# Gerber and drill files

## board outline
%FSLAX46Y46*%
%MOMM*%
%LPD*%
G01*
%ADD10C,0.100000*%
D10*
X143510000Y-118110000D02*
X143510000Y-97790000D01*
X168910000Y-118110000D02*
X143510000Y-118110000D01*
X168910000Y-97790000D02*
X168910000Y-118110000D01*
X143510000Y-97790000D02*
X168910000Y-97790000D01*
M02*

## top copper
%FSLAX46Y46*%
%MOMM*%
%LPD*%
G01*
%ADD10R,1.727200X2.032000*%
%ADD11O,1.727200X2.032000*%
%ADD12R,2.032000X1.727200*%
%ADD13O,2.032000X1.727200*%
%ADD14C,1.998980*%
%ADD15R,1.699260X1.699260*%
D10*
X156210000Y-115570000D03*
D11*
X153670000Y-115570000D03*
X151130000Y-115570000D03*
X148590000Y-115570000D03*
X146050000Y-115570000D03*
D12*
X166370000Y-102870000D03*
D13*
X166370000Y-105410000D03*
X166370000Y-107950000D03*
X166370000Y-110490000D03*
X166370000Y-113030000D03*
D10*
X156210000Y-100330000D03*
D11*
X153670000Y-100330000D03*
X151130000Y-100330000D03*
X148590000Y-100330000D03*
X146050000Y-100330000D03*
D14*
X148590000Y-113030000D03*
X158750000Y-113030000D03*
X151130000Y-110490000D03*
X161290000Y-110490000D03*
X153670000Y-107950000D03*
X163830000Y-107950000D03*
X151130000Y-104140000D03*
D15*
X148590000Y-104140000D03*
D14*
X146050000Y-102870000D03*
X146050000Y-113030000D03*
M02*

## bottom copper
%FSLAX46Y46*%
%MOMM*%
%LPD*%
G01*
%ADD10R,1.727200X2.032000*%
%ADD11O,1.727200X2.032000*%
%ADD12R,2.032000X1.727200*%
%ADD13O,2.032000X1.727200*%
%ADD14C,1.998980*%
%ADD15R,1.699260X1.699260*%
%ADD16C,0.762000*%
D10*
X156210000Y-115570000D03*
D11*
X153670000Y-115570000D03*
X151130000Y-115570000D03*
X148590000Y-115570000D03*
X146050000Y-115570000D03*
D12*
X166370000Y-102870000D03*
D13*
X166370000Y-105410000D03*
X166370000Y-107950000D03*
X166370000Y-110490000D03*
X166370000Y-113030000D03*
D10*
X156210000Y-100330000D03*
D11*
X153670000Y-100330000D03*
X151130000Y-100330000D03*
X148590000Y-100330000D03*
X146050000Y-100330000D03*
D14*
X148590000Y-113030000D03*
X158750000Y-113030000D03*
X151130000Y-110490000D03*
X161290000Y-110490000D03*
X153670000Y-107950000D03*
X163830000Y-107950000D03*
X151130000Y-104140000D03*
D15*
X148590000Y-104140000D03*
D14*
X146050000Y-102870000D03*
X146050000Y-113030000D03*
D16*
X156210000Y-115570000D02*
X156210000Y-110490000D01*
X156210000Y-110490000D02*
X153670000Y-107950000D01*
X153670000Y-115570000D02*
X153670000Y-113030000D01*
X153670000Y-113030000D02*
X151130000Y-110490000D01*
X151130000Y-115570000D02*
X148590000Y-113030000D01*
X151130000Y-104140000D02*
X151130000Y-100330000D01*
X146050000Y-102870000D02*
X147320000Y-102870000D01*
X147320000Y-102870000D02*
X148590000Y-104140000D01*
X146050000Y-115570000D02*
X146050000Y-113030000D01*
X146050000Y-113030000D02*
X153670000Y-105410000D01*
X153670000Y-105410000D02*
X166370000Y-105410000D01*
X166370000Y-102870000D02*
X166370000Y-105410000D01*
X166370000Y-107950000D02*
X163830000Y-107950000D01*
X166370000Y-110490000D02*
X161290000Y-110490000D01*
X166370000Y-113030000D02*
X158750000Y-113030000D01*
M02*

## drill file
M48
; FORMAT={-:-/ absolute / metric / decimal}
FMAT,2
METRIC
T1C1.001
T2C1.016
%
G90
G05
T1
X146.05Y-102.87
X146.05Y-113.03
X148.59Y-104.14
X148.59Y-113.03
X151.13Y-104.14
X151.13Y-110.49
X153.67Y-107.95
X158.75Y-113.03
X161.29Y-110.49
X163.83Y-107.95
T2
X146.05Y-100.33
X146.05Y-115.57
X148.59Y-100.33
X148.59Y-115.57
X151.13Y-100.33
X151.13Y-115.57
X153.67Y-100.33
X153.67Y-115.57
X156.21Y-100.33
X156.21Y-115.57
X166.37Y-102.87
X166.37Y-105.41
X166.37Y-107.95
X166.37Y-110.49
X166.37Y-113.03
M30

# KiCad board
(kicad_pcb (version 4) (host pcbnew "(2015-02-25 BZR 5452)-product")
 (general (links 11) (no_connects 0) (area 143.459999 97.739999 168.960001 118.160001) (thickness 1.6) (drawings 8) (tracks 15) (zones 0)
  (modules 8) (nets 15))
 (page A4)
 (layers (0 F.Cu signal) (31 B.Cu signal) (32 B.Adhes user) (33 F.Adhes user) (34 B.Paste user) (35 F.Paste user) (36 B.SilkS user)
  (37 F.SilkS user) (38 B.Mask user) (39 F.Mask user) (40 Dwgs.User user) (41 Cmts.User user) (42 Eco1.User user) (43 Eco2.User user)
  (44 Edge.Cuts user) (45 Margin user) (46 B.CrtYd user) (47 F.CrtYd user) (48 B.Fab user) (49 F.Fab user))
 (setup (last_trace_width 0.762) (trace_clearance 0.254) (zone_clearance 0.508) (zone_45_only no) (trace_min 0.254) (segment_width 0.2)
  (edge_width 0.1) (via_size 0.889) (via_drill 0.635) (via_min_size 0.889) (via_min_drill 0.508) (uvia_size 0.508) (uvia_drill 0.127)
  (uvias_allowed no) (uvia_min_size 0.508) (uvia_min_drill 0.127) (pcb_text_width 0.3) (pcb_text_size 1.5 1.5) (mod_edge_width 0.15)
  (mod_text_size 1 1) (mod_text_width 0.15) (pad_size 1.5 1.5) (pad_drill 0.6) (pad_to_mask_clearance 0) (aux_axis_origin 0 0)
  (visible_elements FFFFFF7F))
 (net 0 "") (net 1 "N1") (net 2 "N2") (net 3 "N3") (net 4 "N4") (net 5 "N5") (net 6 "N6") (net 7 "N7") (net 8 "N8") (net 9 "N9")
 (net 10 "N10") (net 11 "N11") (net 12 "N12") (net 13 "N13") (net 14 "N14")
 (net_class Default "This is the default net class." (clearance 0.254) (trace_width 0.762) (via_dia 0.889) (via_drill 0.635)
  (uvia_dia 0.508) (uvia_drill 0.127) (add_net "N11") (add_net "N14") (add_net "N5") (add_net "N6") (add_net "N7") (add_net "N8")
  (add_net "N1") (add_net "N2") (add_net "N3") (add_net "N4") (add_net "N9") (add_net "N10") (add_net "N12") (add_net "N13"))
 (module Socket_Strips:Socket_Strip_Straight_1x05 (layer F.Cu) (at 156.21 115.57 180)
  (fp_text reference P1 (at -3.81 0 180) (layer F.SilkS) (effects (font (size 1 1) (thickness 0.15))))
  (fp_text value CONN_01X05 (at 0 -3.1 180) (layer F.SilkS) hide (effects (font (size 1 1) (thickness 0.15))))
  (pad 1 thru_hole rect (at 0 0 180) (size 1.7272 2.032) (drill 1.016) (layers *.Cu *.Mask F.SilkS) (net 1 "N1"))
  (pad 2 thru_hole oval (at 2.54 0 180) (size 1.7272 2.032) (drill 1.016) (layers *.Cu *.Mask F.SilkS) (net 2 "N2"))
  (pad 3 thru_hole oval (at 5.08 0 180) (size 1.7272 2.032) (drill 1.016) (layers *.Cu *.Mask F.SilkS) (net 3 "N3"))
  (pad 4 thru_hole oval (at 7.62 0 180) (size 1.7272 2.032) (drill 1.016) (layers *.Cu *.Mask F.SilkS) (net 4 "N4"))
  (pad 5 thru_hole oval (at 10.16 0 180) (size 1.7272 2.032) (drill 1.016) (layers *.Cu *.Mask F.SilkS) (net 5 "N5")))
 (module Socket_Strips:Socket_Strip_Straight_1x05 (layer F.Cu) (at 166.37 102.87 270)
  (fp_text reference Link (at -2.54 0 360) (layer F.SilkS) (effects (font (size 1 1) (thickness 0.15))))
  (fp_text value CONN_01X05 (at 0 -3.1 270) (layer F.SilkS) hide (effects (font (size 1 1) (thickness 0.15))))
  (pad 1 thru_hole rect (at 0 0 270) (size 1.7272 2.032) (drill 1.016) (layers *.Cu *.Mask F.SilkS) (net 5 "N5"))
  (pad 2 thru_hole oval (at 2.54 0 270) (size 1.7272 2.032) (drill 1.016) (layers *.Cu *.Mask F.SilkS) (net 5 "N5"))
  (pad 3 thru_hole oval (at 5.08 0 270) (size 1.7272 2.032) (drill 1.016) (layers *.Cu *.Mask F.SilkS) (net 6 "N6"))
  (pad 4 thru_hole oval (at 7.62 0 270) (size 1.7272 2.032) (drill 1.016) (layers *.Cu *.Mask F.SilkS) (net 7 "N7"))
  (pad 5 thru_hole oval (at 10.16 0 270) (size 1.7272 2.032) (drill 1.016) (layers *.Cu *.Mask F.SilkS) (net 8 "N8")))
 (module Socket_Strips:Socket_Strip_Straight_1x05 (layer F.Cu) (at 156.21 100.33 180)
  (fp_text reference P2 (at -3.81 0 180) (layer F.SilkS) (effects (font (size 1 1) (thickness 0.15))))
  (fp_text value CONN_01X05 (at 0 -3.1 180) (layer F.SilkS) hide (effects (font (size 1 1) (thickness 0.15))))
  (pad 1 thru_hole rect (at 0 0 180) (size 1.7272 2.032) (drill 1.016) (layers *.Cu *.Mask F.SilkS) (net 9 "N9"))
  (pad 2 thru_hole oval (at 2.54 0 180) (size 1.7272 2.032) (drill 1.016) (layers *.Cu *.Mask F.SilkS) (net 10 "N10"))
  (pad 3 thru_hole oval (at 5.08 0 180) (size 1.7272 2.032) (drill 1.016) (layers *.Cu *.Mask F.SilkS) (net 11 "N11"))
  (pad 4 thru_hole oval (at 7.62 0 180) (size 1.7272 2.032) (drill 1.016) (layers *.Cu *.Mask F.SilkS) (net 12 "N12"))
  (pad 5 thru_hole oval (at 10.16 0 180) (size 1.7272 2.032) (drill 1.016) (layers *.Cu *.Mask F.SilkS) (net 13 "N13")))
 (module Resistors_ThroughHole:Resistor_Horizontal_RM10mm (layer F.Cu) (at 153.67 113.03)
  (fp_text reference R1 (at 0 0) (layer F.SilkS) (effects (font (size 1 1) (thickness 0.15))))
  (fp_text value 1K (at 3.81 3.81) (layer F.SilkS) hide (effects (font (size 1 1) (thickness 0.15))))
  (pad 1 thru_hole circle (at -5.08 0) (size 1.99898 1.99898) (drill 1.00076) (layers *.Cu *.SilkS *.Mask) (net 3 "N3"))
  (pad 2 thru_hole circle (at 5.08 0) (size 1.99898 1.99898) (drill 1.00076) (layers *.Cu *.SilkS *.Mask) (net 8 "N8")))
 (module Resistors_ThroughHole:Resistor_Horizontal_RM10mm (layer F.Cu) (at 156.21 110.49)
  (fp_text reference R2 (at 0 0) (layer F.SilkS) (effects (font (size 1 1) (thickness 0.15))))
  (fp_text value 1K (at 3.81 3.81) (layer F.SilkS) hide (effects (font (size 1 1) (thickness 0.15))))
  (pad 1 thru_hole circle (at -5.08 0) (size 1.99898 1.99898) (drill 1.00076) (layers *.Cu *.SilkS *.Mask) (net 2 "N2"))
  (pad 2 thru_hole circle (at 5.08 0) (size 1.99898 1.99898) (drill 1.00076) (layers *.Cu *.SilkS *.Mask) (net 7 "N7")))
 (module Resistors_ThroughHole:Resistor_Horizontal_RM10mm (layer F.Cu) (at 158.75 107.95)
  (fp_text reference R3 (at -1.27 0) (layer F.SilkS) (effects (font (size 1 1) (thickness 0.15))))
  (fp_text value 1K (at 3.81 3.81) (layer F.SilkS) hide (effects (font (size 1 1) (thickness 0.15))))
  (pad 1 thru_hole circle (at -5.08 0) (size 1.99898 1.99898) (drill 1.00076) (layers *.Cu *.SilkS *.Mask) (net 1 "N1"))
  (pad 2 thru_hole circle (at 5.08 0) (size 1.99898 1.99898) (drill 1.00076) (layers *.Cu *.SilkS *.Mask) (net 6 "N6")))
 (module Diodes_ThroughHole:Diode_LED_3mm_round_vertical (layer F.Cu) (at 149.86 104.14 180)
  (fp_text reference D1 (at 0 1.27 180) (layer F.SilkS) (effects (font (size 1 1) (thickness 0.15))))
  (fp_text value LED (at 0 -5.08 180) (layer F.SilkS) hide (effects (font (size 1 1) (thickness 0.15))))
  (pad 1 thru_hole circle (at -1.27 0 270) (size 1.99898 1.99898) (drill 1.00076) (layers *.Cu *.Mask F.SilkS) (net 11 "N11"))
  (pad 2 thru_hole rect (at 1.27 0 180) (size 1.69926 1.69926) (drill 1.00076) (layers *.Cu *.Mask F.SilkS) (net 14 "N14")))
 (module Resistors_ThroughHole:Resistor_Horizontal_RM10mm (layer F.Cu) (at 146.05 107.95 270)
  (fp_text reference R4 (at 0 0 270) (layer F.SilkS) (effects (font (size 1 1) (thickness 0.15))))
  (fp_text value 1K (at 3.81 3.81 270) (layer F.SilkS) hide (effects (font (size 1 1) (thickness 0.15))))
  (pad 1 thru_hole circle (at -5.08 0 270) (size 1.99898 1.99898) (drill 1.00076) (layers *.Cu *.SilkS *.Mask) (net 14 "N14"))
  (pad 2 thru_hole circle (at 5.08 0 270) (size 1.99898 1.99898) (drill 1.00076) (layers *.Cu *.SilkS *.Mask) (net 5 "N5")))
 (gr_line (start 143.51 118.11) (end 143.51 97.79) (angle 90) (layer Edge.Cuts) (width 0.1))
 (gr_line (start 168.91 118.11) (end 143.51 118.11) (angle 90) (layer Edge.Cuts) (width 0.1))
 (gr_line (start 168.91 97.79) (end 168.91 118.11) (angle 90) (layer Edge.Cuts) (width 0.1))
 (gr_line (start 143.51 97.79) (end 168.91 97.79) (angle 90) (layer Edge.Cuts) (width 0.1))
 (segment (start 156.21 115.57) (end 156.21 110.49) (width 0.762) (layer B.Cu) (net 1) (status 400000))
 (segment (start 156.21 110.49) (end 153.67 107.95) (width 0.762) (layer B.Cu) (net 1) (status 800000))
 (segment (start 153.67 115.57) (end 153.67 113.03) (width 0.762) (layer B.Cu) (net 2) (status 400000))
 (segment (start 153.67 113.03) (end 151.13 110.49) (width 0.762) (layer B.Cu) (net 2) (status 800000))
 (segment (start 151.13 115.57) (end 148.59 113.03) (width 0.762) (layer B.Cu) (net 3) (status C00000))
 (segment (start 151.13 104.14) (end 151.13 100.33) (width 0.762) (layer B.Cu) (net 11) (status C00000))
 (segment (start 146.05 102.87) (end 147.32 102.87) (width 0.762) (layer B.Cu) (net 14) (status 400000))
 (segment (start 147.32 102.87) (end 148.59 104.14) (width 0.762) (layer B.Cu) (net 14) (status 800000))
 (segment (start 146.05 115.57) (end 146.05 113.03) (width 0.762) (layer B.Cu) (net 5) (status C00000))
 (segment (start 146.05 113.03) (end 153.67 105.41) (width 0.762) (layer B.Cu) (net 5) (status 400000))
 (segment (start 153.67 105.41) (end 166.37 105.41) (width 0.762) (layer B.Cu) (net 5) (status 800000))
 (segment (start 166.37 102.87) (end 166.37 105.41) (width 0.762) (layer B.Cu) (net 5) (status C00000))
 (segment (start 166.37 107.95) (end 163.83 107.95) (width 0.762) (layer B.Cu) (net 6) (status C00000))
 (segment (start 166.37 110.49) (end 161.29 110.49) (width 0.762) (layer B.Cu) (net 7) (status C00000))
 (segment (start 166.37 113.03) (end 158.75 113.03) (width 0.762) (layer B.Cu) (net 8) (status C00000)))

